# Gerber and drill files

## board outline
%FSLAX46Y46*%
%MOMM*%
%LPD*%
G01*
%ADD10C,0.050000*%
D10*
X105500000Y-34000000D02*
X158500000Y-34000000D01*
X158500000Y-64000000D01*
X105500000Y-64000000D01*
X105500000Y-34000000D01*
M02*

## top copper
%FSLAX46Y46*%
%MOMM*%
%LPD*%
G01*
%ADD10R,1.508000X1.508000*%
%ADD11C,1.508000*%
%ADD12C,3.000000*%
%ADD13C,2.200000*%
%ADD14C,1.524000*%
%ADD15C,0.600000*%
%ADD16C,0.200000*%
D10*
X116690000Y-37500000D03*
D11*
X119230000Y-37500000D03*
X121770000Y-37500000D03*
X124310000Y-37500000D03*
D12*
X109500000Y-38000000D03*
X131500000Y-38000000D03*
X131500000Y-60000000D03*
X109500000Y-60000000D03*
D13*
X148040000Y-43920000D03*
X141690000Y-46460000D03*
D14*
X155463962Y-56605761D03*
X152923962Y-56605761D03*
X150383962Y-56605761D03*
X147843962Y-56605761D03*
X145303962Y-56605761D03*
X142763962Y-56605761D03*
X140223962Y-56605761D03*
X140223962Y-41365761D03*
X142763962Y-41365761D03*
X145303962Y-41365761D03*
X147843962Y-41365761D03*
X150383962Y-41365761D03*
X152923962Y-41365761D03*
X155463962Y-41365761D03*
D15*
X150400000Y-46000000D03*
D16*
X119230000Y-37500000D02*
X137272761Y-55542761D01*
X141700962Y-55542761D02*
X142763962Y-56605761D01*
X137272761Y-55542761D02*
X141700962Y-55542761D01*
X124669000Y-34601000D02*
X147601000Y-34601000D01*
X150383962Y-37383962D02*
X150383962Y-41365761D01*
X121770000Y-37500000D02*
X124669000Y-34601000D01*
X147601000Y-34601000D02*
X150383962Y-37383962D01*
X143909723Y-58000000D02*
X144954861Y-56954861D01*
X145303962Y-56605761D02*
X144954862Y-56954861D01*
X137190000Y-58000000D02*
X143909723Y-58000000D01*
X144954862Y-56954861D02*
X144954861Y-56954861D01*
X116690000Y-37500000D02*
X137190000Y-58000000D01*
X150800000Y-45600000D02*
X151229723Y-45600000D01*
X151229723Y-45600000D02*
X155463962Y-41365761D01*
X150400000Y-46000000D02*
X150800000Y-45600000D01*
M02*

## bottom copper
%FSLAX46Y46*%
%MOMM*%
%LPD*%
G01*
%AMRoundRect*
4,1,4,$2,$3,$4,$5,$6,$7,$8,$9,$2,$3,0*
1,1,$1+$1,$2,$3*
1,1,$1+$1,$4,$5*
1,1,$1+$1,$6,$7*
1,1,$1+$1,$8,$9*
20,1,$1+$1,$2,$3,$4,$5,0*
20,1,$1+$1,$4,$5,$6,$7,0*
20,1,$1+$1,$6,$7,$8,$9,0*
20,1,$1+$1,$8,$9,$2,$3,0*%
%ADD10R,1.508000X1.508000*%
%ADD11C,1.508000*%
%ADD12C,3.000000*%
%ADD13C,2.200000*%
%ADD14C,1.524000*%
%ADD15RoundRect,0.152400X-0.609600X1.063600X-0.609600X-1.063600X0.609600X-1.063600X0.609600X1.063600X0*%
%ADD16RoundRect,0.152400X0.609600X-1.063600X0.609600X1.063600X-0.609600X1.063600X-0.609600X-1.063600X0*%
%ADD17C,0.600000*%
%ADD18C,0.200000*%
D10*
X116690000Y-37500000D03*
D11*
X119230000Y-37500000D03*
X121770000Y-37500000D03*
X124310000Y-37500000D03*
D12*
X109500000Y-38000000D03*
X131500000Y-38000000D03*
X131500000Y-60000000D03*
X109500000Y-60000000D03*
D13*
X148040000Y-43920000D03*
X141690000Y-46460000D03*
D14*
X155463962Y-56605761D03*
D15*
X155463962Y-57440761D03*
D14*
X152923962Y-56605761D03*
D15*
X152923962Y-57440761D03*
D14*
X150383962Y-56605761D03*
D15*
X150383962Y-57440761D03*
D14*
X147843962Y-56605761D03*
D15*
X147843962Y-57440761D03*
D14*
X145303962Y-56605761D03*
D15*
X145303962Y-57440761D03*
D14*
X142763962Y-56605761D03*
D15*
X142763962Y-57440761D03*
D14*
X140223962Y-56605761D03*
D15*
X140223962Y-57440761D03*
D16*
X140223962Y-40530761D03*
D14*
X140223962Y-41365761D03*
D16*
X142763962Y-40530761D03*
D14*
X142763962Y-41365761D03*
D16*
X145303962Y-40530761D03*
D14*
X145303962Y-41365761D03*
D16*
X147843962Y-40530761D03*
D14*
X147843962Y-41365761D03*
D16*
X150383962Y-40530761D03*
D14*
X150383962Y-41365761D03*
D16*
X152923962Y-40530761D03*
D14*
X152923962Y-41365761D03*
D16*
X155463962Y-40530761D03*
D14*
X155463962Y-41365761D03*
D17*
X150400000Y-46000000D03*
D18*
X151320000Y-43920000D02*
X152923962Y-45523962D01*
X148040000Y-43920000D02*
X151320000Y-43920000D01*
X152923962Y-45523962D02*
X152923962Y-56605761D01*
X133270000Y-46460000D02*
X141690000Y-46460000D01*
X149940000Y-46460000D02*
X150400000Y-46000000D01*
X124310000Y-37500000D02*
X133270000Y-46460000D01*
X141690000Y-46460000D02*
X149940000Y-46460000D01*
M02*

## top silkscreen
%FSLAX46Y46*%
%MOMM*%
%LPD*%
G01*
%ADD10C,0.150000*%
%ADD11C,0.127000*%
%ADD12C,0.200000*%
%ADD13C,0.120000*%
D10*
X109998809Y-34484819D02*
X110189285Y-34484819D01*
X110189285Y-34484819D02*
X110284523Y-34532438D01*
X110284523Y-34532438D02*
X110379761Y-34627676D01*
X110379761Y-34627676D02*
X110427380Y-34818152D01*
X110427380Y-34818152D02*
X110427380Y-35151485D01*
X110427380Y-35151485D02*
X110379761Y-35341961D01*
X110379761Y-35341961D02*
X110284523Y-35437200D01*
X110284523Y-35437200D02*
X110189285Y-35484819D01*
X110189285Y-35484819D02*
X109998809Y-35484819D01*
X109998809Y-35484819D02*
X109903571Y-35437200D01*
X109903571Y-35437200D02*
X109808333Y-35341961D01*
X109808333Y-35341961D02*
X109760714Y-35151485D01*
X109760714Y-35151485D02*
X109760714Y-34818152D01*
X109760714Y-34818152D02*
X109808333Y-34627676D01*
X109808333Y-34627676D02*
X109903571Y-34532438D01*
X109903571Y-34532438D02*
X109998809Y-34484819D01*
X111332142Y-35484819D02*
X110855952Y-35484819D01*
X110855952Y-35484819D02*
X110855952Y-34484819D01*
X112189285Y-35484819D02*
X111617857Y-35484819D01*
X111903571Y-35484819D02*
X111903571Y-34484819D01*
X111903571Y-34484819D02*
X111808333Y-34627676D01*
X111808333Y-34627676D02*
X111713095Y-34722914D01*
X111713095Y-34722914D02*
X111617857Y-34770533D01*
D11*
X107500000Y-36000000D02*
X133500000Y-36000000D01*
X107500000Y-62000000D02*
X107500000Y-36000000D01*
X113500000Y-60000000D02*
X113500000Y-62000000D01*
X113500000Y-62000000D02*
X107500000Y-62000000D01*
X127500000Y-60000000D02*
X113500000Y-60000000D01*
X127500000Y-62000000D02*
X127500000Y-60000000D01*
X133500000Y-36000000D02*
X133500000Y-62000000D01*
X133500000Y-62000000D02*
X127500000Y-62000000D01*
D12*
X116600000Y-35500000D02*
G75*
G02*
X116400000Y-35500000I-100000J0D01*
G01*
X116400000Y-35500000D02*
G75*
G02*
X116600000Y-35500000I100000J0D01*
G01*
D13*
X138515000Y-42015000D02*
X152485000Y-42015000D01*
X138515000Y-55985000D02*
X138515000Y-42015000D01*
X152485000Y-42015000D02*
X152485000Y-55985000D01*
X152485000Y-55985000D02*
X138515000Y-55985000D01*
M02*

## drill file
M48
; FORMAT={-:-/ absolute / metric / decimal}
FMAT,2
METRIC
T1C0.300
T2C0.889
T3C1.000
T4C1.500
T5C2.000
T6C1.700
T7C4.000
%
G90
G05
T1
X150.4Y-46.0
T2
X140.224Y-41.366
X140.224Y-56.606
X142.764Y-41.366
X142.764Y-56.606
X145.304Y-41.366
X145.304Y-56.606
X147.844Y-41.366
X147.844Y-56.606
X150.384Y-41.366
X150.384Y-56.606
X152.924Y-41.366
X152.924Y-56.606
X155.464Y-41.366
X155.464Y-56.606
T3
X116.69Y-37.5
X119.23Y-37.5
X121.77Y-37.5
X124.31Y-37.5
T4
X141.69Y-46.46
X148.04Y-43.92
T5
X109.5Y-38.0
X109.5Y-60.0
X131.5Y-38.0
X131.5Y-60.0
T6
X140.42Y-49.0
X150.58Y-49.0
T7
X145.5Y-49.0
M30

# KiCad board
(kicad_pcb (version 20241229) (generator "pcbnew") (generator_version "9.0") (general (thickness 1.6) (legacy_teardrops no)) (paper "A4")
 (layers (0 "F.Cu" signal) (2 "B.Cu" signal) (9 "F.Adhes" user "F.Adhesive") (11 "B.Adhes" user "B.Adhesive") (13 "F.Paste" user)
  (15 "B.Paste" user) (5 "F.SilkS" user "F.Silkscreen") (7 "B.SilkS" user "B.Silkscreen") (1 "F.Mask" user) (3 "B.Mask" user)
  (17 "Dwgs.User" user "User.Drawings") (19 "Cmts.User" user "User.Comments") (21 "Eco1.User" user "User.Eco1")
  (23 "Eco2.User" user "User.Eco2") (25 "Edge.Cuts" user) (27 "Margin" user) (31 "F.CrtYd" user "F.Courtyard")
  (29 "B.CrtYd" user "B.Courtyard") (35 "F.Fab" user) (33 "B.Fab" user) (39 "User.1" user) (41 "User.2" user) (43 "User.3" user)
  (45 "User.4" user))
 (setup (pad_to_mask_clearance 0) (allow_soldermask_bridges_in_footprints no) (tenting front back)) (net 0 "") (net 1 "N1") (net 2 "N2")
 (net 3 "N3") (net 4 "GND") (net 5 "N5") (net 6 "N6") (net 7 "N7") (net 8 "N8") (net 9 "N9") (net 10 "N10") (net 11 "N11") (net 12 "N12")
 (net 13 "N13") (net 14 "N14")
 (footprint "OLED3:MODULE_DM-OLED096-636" (layer "F.Cu") (at 120.5 49)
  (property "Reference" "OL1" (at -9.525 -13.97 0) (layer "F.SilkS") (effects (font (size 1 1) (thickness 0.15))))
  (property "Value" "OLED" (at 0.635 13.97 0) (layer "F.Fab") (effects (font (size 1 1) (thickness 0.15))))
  (fp_line (start -13 -13) (end 13 -13) (stroke (width 0.127) (type solid)) (layer "F.SilkS"))
  (fp_line (start -13 13) (end -13 -13) (stroke (width 0.127) (type solid)) (layer "F.SilkS"))
  (fp_line (start -7 11) (end -7 13) (stroke (width 0.127) (type solid)) (layer "F.SilkS"))
  (fp_line (start -7 13) (end -13 13) (stroke (width 0.127) (type solid)) (layer "F.SilkS"))
  (fp_line (start 7 11) (end -7 11) (stroke (width 0.127) (type solid)) (layer "F.SilkS"))
  (fp_line (start 7 13) (end 7 11) (stroke (width 0.127) (type solid)) (layer "F.SilkS"))
  (fp_line (start 13 -13) (end 13 13) (stroke (width 0.127) (type solid)) (layer "F.SilkS"))
  (fp_line (start 13 13) (end 7 13) (stroke (width 0.127) (type solid)) (layer "F.SilkS"))
  (fp_circle (center -4 -13.5) (end -3.9 -13.5) (stroke (width 0.2) (type solid)) (fill no) (layer "F.SilkS"))
  (pad "1" thru_hole rect (at -3.81 -11.5) (size 1.508 1.508) (drill 1) (layers "*.Cu" "*.Mask") (remove_unused_layers no) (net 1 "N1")
   (solder_mask_margin 0.102))
  (pad "2" thru_hole circle (at -1.27 -11.5) (size 1.508 1.508) (drill 1) (layers "*.Cu" "*.Mask") (remove_unused_layers no) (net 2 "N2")
   (solder_mask_margin 0.102))
  (pad "3" thru_hole circle (at 1.27 -11.5) (size 1.508 1.508) (drill 1) (layers "*.Cu" "*.Mask") (remove_unused_layers no) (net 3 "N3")
   (solder_mask_margin 0.102))
  (pad "4" thru_hole circle (at 3.81 -11.5) (size 1.508 1.508) (drill 1) (layers "*.Cu" "*.Mask") (remove_unused_layers no) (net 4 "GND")
   (solder_mask_margin 0.102))
  (pad "S1" thru_hole circle (at -11 -11) (size 3 3) (drill 2) (layers "*.Cu" "*.Mask") (remove_unused_layers no) (solder_mask_margin 0.102))
  (pad "S2" thru_hole circle (at 11 -11) (size 3 3) (drill 2) (layers "*.Cu" "*.Mask") (remove_unused_layers no) (solder_mask_margin 0.102))
  (pad "S3" thru_hole circle (at 11 11) (size 3 3) (drill 2) (layers "*.Cu" "*.Mask") (remove_unused_layers no) (solder_mask_margin 0.102))
  (pad "S4" thru_hole circle (at -11 11) (size 3 3) (drill 2) (layers "*.Cu" "*.Mask") (remove_unused_layers no) (solder_mask_margin 0.102)))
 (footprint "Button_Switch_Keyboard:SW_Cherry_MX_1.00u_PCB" (layer "F.Cu") (at 148.04 43.92)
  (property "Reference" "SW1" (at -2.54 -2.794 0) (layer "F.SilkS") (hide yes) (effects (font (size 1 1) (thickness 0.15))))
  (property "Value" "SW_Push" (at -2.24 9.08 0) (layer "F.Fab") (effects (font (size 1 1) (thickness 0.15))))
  (fp_line (start -9.525 -1.905) (end 4.445 -1.905) (stroke (width 0.12) (type solid)) (layer "F.SilkS"))
  (fp_line (start -9.525 12.065) (end -9.525 -1.905) (stroke (width 0.12) (type solid)) (layer "F.SilkS"))
  (fp_line (start 4.445 -1.905) (end 4.445 12.065) (stroke (width 0.12) (type solid)) (layer "F.SilkS"))
  (fp_line (start 4.445 12.065) (end -9.525 12.065) (stroke (width 0.12) (type solid)) (layer "F.SilkS"))
  (pad "" np_thru_hole circle (at -7.62 5.08) (size 1.7 1.7) (drill 1.7) (layers "*.Cu" "*.Mask"))
  (pad "" np_thru_hole circle (at -2.54 5.08) (size 4 4) (drill 4) (layers "*.Cu" "*.Mask"))
  (pad "" np_thru_hole circle (at 2.54 5.08) (size 1.7 1.7) (drill 1.7) (layers "*.Cu" "*.Mask"))
  (pad "1" thru_hole circle (at 0 0) (size 2.2 2.2) (drill 1.5) (layers "*.Cu" "*.Mask") (remove_unused_layers no) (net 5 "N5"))
  (pad "2" thru_hole circle (at -6.35 2.54) (size 2.2 2.2) (drill 1.5) (layers "*.Cu" "*.Mask") (remove_unused_layers no) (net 4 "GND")))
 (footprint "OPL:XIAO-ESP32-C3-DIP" (layer "B.Cu") (at 147.843962 48.985761)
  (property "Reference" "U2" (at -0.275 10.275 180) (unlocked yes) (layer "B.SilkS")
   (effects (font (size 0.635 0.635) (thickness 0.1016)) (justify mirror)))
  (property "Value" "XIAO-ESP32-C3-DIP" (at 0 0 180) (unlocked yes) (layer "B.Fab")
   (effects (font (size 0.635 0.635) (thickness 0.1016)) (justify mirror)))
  (pad "1" thru_hole circle (at 7.62 7.62 270) (size 1.524 1.524) (drill 0.889) (layers "*.Cu" "*.Mask") (remove_unused_layers no)
   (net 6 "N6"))
  (pad "1" smd roundrect (at 7.62 8.455 270) (size 2.432 1.524) (layers "B.Cu" "B.Mask") (roundrect_rratio 0.1) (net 6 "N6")
   (thermal_bridge_angle 45))
  (pad "2" thru_hole circle (at 5.08 7.62 270) (size 1.524 1.524) (drill 0.889) (layers "*.Cu" "*.Mask") (remove_unused_layers no)
   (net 5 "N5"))
  (pad "2" smd roundrect (at 5.08 8.455 270) (size 2.432 1.524) (layers "B.Cu" "B.Mask") (roundrect_rratio 0.1) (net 5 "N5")
   (thermal_bridge_angle 45))
  (pad "3" thru_hole circle (at 2.54 7.62 270) (size 1.524 1.524) (drill 0.889) (layers "*.Cu" "*.Mask") (remove_unused_layers no)
   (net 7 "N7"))
  (pad "3" smd roundrect (at 2.54 8.455 270) (size 2.432 1.524) (layers "B.Cu" "B.Mask") (roundrect_rratio 0.1) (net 7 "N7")
   (thermal_bridge_angle 45))
  (pad "4" thru_hole circle (at 0 7.62 270) (size 1.524 1.524) (drill 0.889) (layers "*.Cu" "*.Mask") (remove_unused_layers no) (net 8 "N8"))
  (pad "4" smd roundrect (at 0 8.455 270) (size 2.432 1.524) (layers "B.Cu" "B.Mask") (roundrect_rratio 0.1) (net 8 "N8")
   (thermal_bridge_angle 45))
  (pad "5" thru_hole circle (at -2.54 7.62 270) (size 1.524 1.524) (drill 0.889) (layers "*.Cu" "*.Mask") (remove_unused_layers no)
   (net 1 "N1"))
  (pad "5" smd roundrect (at -2.54 8.455 270) (size 2.432 1.524) (layers "B.Cu" "B.Mask") (roundrect_rratio 0.1) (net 1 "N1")
   (thermal_bridge_angle 45))
  (pad "6" thru_hole circle (at -5.08 7.62 270) (size 1.524 1.524) (drill 0.889) (layers "*.Cu" "*.Mask") (remove_unused_layers no)
   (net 2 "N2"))
  (pad "6" smd roundrect (at -5.08 8.455 270) (size 2.432 1.524) (layers "B.Cu" "B.Mask") (roundrect_rratio 0.1) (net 2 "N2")
   (thermal_bridge_angle 45))
  (pad "7" thru_hole circle (at -7.62 7.62 270) (size 1.524 1.524) (drill 0.889) (layers "*.Cu" "*.Mask") (remove_unused_layers no)
   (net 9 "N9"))
  (pad "7" smd roundrect (at -7.62 8.455 270) (size 2.432 1.524) (layers "B.Cu" "B.Mask") (roundrect_rratio 0.1) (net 9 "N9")
   (thermal_bridge_angle 45))
  (pad "8" smd roundrect (at -7.62 -8.455 90) (size 2.432 1.524) (layers "B.Cu" "B.Mask") (roundrect_rratio 0.1) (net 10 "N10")
   (thermal_bridge_angle 45))
  (pad "8" thru_hole circle (at -7.62 -7.62 90) (size 1.524 1.524) (drill 0.889) (layers "*.Cu" "*.Mask") (remove_unused_layers no)
   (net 10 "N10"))
  (pad "9" smd roundrect (at -5.08 -8.455 90) (size 2.432 1.524) (layers "B.Cu" "B.Mask") (roundrect_rratio 0.1) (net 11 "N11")
   (thermal_bridge_angle 45))
  (pad "9" thru_hole circle (at -5.08 -7.62 90) (size 1.524 1.524) (drill 0.889) (layers "*.Cu" "*.Mask") (remove_unused_layers no)
   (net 11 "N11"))
  (pad "10" smd roundrect (at -2.54 -8.455 90) (size 2.432 1.524) (layers "B.Cu" "B.Mask") (roundrect_rratio 0.1) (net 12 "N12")
   (thermal_bridge_angle 45))
  (pad "10" thru_hole circle (at -2.54 -7.62 90) (size 1.524 1.524) (drill 0.889) (layers "*.Cu" "*.Mask") (remove_unused_layers no)
   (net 12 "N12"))
  (pad "11" smd roundrect (at 0 -8.455 90) (size 2.432 1.524) (layers "B.Cu" "B.Mask") (roundrect_rratio 0.1) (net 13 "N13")
   (thermal_bridge_angle 45))
  (pad "11" thru_hole circle (at 0 -7.62 90) (size 1.524 1.524) (drill 0.889) (layers "*.Cu" "*.Mask") (remove_unused_layers no)
   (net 13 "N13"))
  (pad "12" smd roundrect (at 2.54 -8.455 90) (size 2.432 1.524) (layers "B.Cu" "B.Mask") (roundrect_rratio 0.1) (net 3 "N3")
   (thermal_bridge_angle 45))
  (pad "12" thru_hole circle (at 2.54 -7.62 90) (size 1.524 1.524) (drill 0.889) (layers "*.Cu" "*.Mask") (remove_unused_layers no)
   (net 3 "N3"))
  (pad "13" smd roundrect (at 5.08 -8.455 90) (size 2.432 1.524) (layers "B.Cu" "B.Mask") (roundrect_rratio 0.1) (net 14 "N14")
   (thermal_bridge_angle 45))
  (pad "13" thru_hole circle (at 5.08 -7.62 90) (size 1.524 1.524) (drill 0.889) (layers "*.Cu" "*.Mask") (remove_unused_layers no)
   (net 14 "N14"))
  (pad "14" smd roundrect (at 7.62 -8.455 90) (size 2.432 1.524) (layers "B.Cu" "B.Mask") (roundrect_rratio 0.1) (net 4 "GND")
   (thermal_bridge_angle 45))
  (pad "14" thru_hole circle (at 7.62 -7.62 90) (size 1.524 1.524) (drill 0.889) (layers "*.Cu" "*.Mask") (remove_unused_layers no)
   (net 4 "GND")))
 (gr_rect (start 105.5 34) (end 158.5 64) (stroke (width 0.05) (type default)) (fill no) (layer "Edge.Cuts"))
 (segment (start 119.23 37.5) (end 137.272761 55.542761) (width 0.2) (layer "F.Cu") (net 2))
 (segment (start 141.700962 55.542761) (end 142.763962 56.605761) (width 0.2) (layer "F.Cu") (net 2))
 (segment (start 137.272761 55.542761) (end 141.700962 55.542761) (width 0.2) (layer "F.Cu") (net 2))
 (segment (start 124.669 34.601) (end 147.601 34.601) (width 0.2) (layer "F.Cu") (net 3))
 (segment (start 150.383962 37.383962) (end 150.383962 41.365761) (width 0.2) (layer "F.Cu") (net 3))
 (segment (start 121.77 37.5) (end 124.669 34.601) (width 0.2) (layer "F.Cu") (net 3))
 (segment (start 147.601 34.601) (end 150.383962 37.383962) (width 0.2) (layer "F.Cu") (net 3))
 (segment (start 143.909723 58) (end 144.954861 56.954861) (width 0.2) (layer "F.Cu") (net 1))
 (segment (start 145.303962 56.605761) (end 144.954862 56.954861) (width 0.2) (layer "F.Cu") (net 1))
 (segment (start 137.19 58) (end 143.909723 58) (width 0.2) (layer "F.Cu") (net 1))
 (segment (start 144.954862 56.954861) (end 144.954861 56.954861) (width 0.2) (layer "F.Cu") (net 1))
 (segment (start 116.69 37.5) (end 137.19 58) (width 0.2) (layer "F.Cu") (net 1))
 (segment (start 151.32 43.92) (end 152.923962 45.523962) (width 0.2) (layer "B.Cu") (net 5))
 (segment (start 148.04 43.92) (end 151.32 43.92) (width 0.2) (layer "B.Cu") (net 5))
 (segment (start 152.923962 45.523962) (end 152.923962 56.605761) (width 0.2) (layer "B.Cu") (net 5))
 (segment (start 150.8 45.6) (end 151.229723 45.6) (width 0.2) (layer "F.Cu") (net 4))
 (segment (start 151.229723 45.6) (end 155.463962 41.365761) (width 0.2) (layer "F.Cu") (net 4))
 (segment (start 150.4 46) (end 150.8 45.6) (width 0.2) (layer "F.Cu") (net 4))
 (via (at 150.4 46) (size 0.6) (drill 0.3) (layers "F.Cu" "B.Cu") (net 4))
 (segment (start 133.27 46.46) (end 141.69 46.46) (width 0.2) (layer "B.Cu") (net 4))
 (segment (start 149.94 46.46) (end 150.4 46) (width 0.2) (layer "B.Cu") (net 4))
 (segment (start 124.31 37.5) (end 133.27 46.46) (width 0.2) (layer "B.Cu") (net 4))
 (segment (start 141.69 46.46) (end 149.94 46.46) (width 0.2) (layer "B.Cu") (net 4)))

